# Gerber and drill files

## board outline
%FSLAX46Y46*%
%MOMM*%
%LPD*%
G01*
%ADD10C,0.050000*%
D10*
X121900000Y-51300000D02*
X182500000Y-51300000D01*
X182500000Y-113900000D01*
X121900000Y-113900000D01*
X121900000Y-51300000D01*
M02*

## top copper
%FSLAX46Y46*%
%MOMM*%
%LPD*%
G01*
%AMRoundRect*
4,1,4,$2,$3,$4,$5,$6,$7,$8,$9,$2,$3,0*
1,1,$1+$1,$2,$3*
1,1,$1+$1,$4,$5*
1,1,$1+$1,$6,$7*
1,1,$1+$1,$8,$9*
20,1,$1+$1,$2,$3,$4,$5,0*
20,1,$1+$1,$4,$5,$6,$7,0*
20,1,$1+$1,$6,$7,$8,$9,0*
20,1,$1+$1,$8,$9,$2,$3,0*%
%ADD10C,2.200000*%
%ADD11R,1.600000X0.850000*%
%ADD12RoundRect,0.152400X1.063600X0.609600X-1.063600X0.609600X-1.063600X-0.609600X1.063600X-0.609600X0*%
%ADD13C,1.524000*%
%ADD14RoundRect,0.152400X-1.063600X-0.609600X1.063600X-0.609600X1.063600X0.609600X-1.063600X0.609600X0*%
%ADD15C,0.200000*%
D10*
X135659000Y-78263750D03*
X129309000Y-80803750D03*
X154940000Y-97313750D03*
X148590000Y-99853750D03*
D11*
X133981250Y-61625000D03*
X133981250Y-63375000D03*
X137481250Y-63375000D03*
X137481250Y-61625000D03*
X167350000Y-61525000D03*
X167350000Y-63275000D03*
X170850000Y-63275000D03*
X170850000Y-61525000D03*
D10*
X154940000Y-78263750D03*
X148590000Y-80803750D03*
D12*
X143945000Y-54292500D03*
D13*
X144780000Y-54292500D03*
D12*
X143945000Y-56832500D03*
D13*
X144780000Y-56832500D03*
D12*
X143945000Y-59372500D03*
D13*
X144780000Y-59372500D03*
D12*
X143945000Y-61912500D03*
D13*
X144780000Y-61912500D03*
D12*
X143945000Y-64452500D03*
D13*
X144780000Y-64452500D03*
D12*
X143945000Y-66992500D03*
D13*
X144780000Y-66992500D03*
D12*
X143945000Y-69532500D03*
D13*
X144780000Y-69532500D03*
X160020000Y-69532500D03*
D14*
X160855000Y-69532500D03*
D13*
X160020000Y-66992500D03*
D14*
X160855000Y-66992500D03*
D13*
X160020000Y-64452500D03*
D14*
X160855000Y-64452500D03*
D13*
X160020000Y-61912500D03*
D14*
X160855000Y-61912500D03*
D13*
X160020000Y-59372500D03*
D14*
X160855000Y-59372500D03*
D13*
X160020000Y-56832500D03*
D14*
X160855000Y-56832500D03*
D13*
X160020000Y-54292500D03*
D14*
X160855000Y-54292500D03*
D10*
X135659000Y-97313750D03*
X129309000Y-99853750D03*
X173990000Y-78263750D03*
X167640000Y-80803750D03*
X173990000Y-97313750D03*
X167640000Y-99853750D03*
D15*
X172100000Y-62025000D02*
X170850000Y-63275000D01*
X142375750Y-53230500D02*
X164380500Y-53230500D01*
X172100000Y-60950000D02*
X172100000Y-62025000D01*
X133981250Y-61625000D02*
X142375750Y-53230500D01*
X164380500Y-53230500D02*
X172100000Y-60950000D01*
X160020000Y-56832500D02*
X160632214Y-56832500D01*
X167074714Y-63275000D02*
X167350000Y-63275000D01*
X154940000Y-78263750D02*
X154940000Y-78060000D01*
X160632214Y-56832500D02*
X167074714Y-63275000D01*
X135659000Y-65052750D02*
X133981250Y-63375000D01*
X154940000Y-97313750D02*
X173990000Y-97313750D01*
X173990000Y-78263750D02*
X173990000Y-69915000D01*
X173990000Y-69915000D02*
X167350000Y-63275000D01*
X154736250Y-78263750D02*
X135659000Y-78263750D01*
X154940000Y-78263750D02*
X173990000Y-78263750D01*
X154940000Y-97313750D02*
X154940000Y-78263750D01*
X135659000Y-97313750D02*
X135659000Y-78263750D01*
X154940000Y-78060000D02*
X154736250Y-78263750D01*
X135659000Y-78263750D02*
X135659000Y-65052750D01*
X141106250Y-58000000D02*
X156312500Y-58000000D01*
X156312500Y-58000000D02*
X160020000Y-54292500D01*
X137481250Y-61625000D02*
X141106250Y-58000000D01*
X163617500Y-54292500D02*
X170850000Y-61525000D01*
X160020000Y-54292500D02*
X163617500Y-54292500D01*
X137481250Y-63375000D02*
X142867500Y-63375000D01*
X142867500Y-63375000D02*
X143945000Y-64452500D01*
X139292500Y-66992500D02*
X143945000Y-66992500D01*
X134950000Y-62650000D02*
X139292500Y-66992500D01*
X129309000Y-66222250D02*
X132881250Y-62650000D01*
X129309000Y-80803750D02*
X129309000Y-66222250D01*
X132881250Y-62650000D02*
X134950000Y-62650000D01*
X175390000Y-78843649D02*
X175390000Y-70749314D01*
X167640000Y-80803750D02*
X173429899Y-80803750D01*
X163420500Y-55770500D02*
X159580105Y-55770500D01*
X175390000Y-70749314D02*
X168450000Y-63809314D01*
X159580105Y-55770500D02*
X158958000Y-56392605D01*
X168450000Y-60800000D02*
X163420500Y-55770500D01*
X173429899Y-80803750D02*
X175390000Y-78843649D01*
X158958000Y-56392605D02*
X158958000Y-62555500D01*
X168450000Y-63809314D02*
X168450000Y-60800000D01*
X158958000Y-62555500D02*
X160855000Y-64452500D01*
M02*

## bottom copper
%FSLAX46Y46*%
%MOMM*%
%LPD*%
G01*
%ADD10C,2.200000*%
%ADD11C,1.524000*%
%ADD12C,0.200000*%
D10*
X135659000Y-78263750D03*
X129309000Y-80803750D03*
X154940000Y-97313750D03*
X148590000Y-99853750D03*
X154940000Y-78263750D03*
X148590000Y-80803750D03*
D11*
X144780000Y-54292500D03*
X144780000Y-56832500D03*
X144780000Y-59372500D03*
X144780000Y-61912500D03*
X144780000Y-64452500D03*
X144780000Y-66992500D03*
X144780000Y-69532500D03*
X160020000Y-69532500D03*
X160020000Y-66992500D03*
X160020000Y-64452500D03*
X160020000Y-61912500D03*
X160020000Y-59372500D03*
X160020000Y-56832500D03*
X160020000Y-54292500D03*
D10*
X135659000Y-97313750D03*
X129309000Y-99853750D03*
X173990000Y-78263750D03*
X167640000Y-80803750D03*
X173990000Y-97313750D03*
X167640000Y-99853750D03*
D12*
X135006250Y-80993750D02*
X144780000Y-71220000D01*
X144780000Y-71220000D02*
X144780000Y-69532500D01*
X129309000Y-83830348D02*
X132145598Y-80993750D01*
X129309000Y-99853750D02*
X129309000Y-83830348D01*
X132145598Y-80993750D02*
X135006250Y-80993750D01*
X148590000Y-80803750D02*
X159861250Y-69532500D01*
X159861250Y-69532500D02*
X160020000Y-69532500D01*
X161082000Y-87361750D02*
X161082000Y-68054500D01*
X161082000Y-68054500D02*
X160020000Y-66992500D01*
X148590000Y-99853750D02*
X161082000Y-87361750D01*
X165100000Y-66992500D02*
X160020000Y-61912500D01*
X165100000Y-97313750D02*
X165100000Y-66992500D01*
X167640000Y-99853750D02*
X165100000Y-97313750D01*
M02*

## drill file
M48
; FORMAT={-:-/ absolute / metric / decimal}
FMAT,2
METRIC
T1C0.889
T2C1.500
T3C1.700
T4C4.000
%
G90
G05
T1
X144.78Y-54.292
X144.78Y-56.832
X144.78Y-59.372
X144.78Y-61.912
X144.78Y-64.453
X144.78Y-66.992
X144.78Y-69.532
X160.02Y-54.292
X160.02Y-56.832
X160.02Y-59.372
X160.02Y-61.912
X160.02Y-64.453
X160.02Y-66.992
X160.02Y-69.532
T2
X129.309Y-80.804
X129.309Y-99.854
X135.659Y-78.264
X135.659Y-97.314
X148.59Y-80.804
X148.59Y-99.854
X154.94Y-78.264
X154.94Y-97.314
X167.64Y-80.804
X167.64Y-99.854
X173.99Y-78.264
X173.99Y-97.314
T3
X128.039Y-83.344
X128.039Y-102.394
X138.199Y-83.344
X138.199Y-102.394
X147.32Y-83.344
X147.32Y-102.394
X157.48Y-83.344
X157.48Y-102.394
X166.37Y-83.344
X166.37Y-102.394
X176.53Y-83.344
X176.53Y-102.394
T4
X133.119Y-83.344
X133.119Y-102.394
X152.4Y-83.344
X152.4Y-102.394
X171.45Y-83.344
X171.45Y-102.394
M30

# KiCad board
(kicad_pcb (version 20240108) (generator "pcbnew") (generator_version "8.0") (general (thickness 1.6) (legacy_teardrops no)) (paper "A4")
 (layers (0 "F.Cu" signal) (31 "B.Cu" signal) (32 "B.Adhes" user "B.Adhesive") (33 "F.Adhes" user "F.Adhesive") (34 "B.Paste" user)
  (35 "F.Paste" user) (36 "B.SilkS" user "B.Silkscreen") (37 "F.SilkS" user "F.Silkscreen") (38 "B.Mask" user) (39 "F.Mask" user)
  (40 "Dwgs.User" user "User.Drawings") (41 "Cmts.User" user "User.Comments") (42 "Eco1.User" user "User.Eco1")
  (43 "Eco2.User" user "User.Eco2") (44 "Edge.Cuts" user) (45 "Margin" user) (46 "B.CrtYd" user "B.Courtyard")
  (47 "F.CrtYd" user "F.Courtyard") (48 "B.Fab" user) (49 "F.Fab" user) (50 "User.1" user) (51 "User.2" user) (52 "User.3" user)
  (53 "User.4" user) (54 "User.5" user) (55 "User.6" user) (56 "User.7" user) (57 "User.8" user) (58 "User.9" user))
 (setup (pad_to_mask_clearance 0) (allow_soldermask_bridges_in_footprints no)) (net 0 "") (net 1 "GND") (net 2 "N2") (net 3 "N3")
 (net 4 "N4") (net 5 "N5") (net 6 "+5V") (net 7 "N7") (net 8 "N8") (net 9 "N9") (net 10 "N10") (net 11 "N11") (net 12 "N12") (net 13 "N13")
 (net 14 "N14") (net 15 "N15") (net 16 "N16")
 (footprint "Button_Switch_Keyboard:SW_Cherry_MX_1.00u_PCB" (layer "F.Cu") (at 135.659 78.26375)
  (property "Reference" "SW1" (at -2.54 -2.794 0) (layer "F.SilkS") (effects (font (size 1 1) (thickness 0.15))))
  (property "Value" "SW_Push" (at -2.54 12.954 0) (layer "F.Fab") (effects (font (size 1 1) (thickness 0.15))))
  (pad "" np_thru_hole circle (at -7.62 5.08) (size 1.7 1.7) (drill 1.7) (layers "*.Cu" "*.Mask"))
  (pad "" np_thru_hole circle (at -2.54 5.08) (size 4 4) (drill 4) (layers "*.Cu" "*.Mask"))
  (pad "" np_thru_hole circle (at 2.54 5.08) (size 1.7 1.7) (drill 1.7) (layers "*.Cu" "*.Mask"))
  (pad "1" thru_hole circle (at 0 0) (size 2.2 2.2) (drill 1.5) (layers "*.Cu" "*.Mask") (remove_unused_layers no) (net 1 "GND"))
  (pad "2" thru_hole circle (at -6.35 2.54) (size 2.2 2.2) (drill 1.5) (layers "*.Cu" "*.Mask") (remove_unused_layers no) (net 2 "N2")))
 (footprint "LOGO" (layer "F.Cu") (at 153.1 80.9)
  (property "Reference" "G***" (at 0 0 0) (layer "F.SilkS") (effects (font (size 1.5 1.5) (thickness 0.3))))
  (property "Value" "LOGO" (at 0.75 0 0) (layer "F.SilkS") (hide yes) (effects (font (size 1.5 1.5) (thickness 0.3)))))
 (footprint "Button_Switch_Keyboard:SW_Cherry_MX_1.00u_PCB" (layer "F.Cu") (at 154.94 97.31375)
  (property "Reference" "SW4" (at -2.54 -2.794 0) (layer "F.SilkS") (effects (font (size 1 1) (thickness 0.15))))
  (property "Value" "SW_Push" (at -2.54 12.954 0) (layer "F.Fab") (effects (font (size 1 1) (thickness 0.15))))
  (pad "" np_thru_hole circle (at -7.62 5.08) (size 1.7 1.7) (drill 1.7) (layers "*.Cu" "*.Mask"))
  (pad "" np_thru_hole circle (at -2.54 5.08) (size 4 4) (drill 4) (layers "*.Cu" "*.Mask"))
  (pad "" np_thru_hole circle (at 2.54 5.08) (size 1.7 1.7) (drill 1.7) (layers "*.Cu" "*.Mask"))
  (pad "1" thru_hole circle (at 0 0) (size 2.2 2.2) (drill 1.5) (layers "*.Cu" "*.Mask") (remove_unused_layers no) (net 1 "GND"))
  (pad "2" thru_hole circle (at -6.35 2.54) (size 2.2 2.2) (drill 1.5) (layers "*.Cu" "*.Mask") (remove_unused_layers no) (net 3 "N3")))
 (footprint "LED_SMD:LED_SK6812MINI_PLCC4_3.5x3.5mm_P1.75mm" (layer "F.Cu") (at 135.73125 62.5)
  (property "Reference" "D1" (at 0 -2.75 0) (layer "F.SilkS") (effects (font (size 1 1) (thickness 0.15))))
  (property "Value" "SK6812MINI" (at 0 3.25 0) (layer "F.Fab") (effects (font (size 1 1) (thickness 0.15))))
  (pad "1" smd rect (at -1.75 -0.875) (size 1.6 0.85) (layers "F.Cu" "F.Paste" "F.Mask") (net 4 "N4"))
  (pad "2" smd rect (at -1.75 0.875) (size 1.6 0.85) (layers "F.Cu" "F.Paste" "F.Mask") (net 1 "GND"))
  (pad "3" smd rect (at 1.75 0.875) (size 1.6 0.85) (layers "F.Cu" "F.Paste" "F.Mask") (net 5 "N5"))
  (pad "4" smd rect (at 1.75 -0.875) (size 1.6 0.85) (layers "F.Cu" "F.Paste" "F.Mask") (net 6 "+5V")))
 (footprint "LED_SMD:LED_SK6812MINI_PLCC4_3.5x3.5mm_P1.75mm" (layer "F.Cu") (at 169.1 62.4)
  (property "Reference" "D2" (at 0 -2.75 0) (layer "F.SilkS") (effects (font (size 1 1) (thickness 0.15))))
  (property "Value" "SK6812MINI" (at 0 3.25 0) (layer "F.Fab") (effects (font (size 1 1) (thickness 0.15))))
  (pad "1" smd rect (at -1.75 -0.875) (size 1.6 0.85) (layers "F.Cu" "F.Paste" "F.Mask") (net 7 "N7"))
  (pad "2" smd rect (at -1.75 0.875) (size 1.6 0.85) (layers "F.Cu" "F.Paste" "F.Mask") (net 1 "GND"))
  (pad "3" smd rect (at 1.75 0.875) (size 1.6 0.85) (layers "F.Cu" "F.Paste" "F.Mask") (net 4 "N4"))
  (pad "4" smd rect (at 1.75 -0.875) (size 1.6 0.85) (layers "F.Cu" "F.Paste" "F.Mask") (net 6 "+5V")))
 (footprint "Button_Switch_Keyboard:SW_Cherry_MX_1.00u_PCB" (layer "F.Cu") (at 154.94 78.26375)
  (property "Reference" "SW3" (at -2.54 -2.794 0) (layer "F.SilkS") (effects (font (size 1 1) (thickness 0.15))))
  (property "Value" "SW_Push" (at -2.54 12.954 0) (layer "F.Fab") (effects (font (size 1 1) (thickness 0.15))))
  (pad "" np_thru_hole circle (at -7.62 5.08) (size 1.7 1.7) (drill 1.7) (layers "*.Cu" "*.Mask"))
  (pad "" np_thru_hole circle (at -2.54 5.08) (size 4 4) (drill 4) (layers "*.Cu" "*.Mask"))
  (pad "" np_thru_hole circle (at 2.54 5.08) (size 1.7 1.7) (drill 1.7) (layers "*.Cu" "*.Mask"))
  (pad "1" thru_hole circle (at 0 0) (size 2.2 2.2) (drill 1.5) (layers "*.Cu" "*.Mask") (remove_unused_layers no) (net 1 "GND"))
  (pad "2" thru_hole circle (at -6.35 2.54) (size 2.2 2.2) (drill 1.5) (layers "*.Cu" "*.Mask") (remove_unused_layers no) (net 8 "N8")))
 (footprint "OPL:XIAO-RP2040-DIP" (layer "F.Cu") (at 152.4 61.9125)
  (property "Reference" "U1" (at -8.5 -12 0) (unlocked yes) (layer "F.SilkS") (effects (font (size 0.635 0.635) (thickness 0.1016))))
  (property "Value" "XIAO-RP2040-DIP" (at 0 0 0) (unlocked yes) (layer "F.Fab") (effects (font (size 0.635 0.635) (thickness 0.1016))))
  (pad "1" smd roundrect (at -8.455 -7.62 180) (size 2.432 1.524) (layers "F.Cu" "F.Mask") (roundrect_rratio 0.1) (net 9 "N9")
   (thermal_bridge_angle 45))
  (pad "1" thru_hole circle (at -7.62 -7.62 180) (size 1.524 1.524) (drill 0.889) (layers "*.Cu" "*.Mask") (remove_unused_layers no)
   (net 9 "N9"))
  (pad "2" smd roundrect (at -8.455 -5.08 180) (size 2.432 1.524) (layers "F.Cu" "F.Mask") (roundrect_rratio 0.1) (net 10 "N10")
   (thermal_bridge_angle 45))
  (pad "2" thru_hole circle (at -7.62 -5.08 180) (size 1.524 1.524) (drill 0.889) (layers "*.Cu" "*.Mask") (remove_unused_layers no)
   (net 10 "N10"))
  (pad "3" smd roundrect (at -8.455 -2.54 180) (size 2.432 1.524) (layers "F.Cu" "F.Mask") (roundrect_rratio 0.1) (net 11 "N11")
   (thermal_bridge_angle 45))
  (pad "3" thru_hole circle (at -7.62 -2.54 180) (size 1.524 1.524) (drill 0.889) (layers "*.Cu" "*.Mask") (remove_unused_layers no)
   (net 11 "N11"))
  (pad "4" smd roundrect (at -8.455 0 180) (size 2.432 1.524) (layers "F.Cu" "F.Mask") (roundrect_rratio 0.1) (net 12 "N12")
   (thermal_bridge_angle 45))
  (pad "4" thru_hole circle (at -7.62 0 180) (size 1.524 1.524) (drill 0.889) (layers "*.Cu" "*.Mask") (remove_unused_layers no)
   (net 12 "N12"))
  (pad "5" smd roundrect (at -8.455 2.54 180) (size 2.432 1.524) (layers "F.Cu" "F.Mask") (roundrect_rratio 0.1) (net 5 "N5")
   (thermal_bridge_angle 45))
  (pad "5" thru_hole circle (at -7.62 2.54 180) (size 1.524 1.524) (drill 0.889) (layers "*.Cu" "*.Mask") (remove_unused_layers no)
   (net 5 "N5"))
  (pad "6" smd roundrect (at -8.455 5.08 180) (size 2.432 1.524) (layers "F.Cu" "F.Mask") (roundrect_rratio 0.1) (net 2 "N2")
   (thermal_bridge_angle 45))
  (pad "6" thru_hole circle (at -7.62 5.08 180) (size 1.524 1.524) (drill 0.889) (layers "*.Cu" "*.Mask") (remove_unused_layers no)
   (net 2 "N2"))
  (pad "7" smd roundrect (at -8.455 7.62 180) (size 2.432 1.524) (layers "F.Cu" "F.Mask") (roundrect_rratio 0.1) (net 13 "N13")
   (thermal_bridge_angle 45))
  (pad "7" thru_hole circle (at -7.62 7.62 180) (size 1.524 1.524) (drill 0.889) (layers "*.Cu" "*.Mask") (remove_unused_layers no)
   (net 13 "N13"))
  (pad "8" thru_hole circle (at 7.62 7.62) (size 1.524 1.524) (drill 0.889) (layers "*.Cu" "*.Mask") (remove_unused_layers no) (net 8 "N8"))
  (pad "8" smd roundrect (at 8.455 7.62) (size 2.432 1.524) (layers "F.Cu" "F.Mask") (roundrect_rratio 0.1) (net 8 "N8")
   (thermal_bridge_angle 45))
  (pad "9" thru_hole circle (at 7.62 5.08) (size 1.524 1.524) (drill 0.889) (layers "*.Cu" "*.Mask") (remove_unused_layers no) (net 3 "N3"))
  (pad "9" smd roundrect (at 8.455 5.08) (size 2.432 1.524) (layers "F.Cu" "F.Mask") (roundrect_rratio 0.1) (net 3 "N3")
   (thermal_bridge_angle 45))
  (pad "10" thru_hole circle (at 7.62 2.54) (size 1.524 1.524) (drill 0.889) (layers "*.Cu" "*.Mask") (remove_unused_layers no)
   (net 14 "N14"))
  (pad "10" smd roundrect (at 8.455 2.54) (size 2.432 1.524) (layers "F.Cu" "F.Mask") (roundrect_rratio 0.1) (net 14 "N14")
   (thermal_bridge_angle 45))
  (pad "11" thru_hole circle (at 7.62 0) (size 1.524 1.524) (drill 0.889) (layers "*.Cu" "*.Mask") (remove_unused_layers no) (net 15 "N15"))
  (pad "11" smd roundrect (at 8.455 0) (size 2.432 1.524) (layers "F.Cu" "F.Mask") (roundrect_rratio 0.1) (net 15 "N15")
   (thermal_bridge_angle 45))
  (pad "12" thru_hole circle (at 7.62 -2.54) (size 1.524 1.524) (drill 0.889) (layers "*.Cu" "*.Mask") (remove_unused_layers no)
   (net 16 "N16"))
  (pad "12" smd roundrect (at 8.455 -2.54) (size 2.432 1.524) (layers "F.Cu" "F.Mask") (roundrect_rratio 0.1) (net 16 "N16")
   (thermal_bridge_angle 45))
  (pad "13" thru_hole circle (at 7.62 -5.08) (size 1.524 1.524) (drill 0.889) (layers "*.Cu" "*.Mask") (remove_unused_layers no)
   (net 1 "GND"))
  (pad "13" smd roundrect (at 8.455 -5.08) (size 2.432 1.524) (layers "F.Cu" "F.Mask") (roundrect_rratio 0.1) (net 1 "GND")
   (thermal_bridge_angle 45))
  (pad "14" thru_hole circle (at 7.62 -7.62) (size 1.524 1.524) (drill 0.889) (layers "*.Cu" "*.Mask") (remove_unused_layers no)
   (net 6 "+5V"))
  (pad "14" smd roundrect (at 8.455 -7.62) (size 2.432 1.524) (layers "F.Cu" "F.Mask") (roundrect_rratio 0.1) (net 6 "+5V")
   (thermal_bridge_angle 45)))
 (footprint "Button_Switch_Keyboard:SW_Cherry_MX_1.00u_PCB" (layer "F.Cu") (at 135.659 97.31375)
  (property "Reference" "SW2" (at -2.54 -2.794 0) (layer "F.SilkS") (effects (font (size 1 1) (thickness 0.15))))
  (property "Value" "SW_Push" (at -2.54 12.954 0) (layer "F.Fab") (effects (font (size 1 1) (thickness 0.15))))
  (pad "" np_thru_hole circle (at -7.62 5.08) (size 1.7 1.7) (drill 1.7) (layers "*.Cu" "*.Mask"))
  (pad "" np_thru_hole circle (at -2.54 5.08) (size 4 4) (drill 4) (layers "*.Cu" "*.Mask"))
  (pad "" np_thru_hole circle (at 2.54 5.08) (size 1.7 1.7) (drill 1.7) (layers "*.Cu" "*.Mask"))
  (pad "1" thru_hole circle (at 0 0) (size 2.2 2.2) (drill 1.5) (layers "*.Cu" "*.Mask") (remove_unused_layers no) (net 1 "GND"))
  (pad "2" thru_hole circle (at -6.35 2.54) (size 2.2 2.2) (drill 1.5) (layers "*.Cu" "*.Mask") (remove_unused_layers no) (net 13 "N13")))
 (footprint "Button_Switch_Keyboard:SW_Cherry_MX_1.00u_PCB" (layer "F.Cu") (at 173.99 78.26375)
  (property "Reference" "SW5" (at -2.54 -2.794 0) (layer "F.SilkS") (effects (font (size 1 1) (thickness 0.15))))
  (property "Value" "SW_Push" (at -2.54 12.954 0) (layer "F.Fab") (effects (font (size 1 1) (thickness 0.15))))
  (pad "" np_thru_hole circle (at -7.62 5.08) (size 1.7 1.7) (drill 1.7) (layers "*.Cu" "*.Mask"))
  (pad "" np_thru_hole circle (at -2.54 5.08) (size 4 4) (drill 4) (layers "*.Cu" "*.Mask"))
  (pad "" np_thru_hole circle (at 2.54 5.08) (size 1.7 1.7) (drill 1.7) (layers "*.Cu" "*.Mask"))
  (pad "1" thru_hole circle (at 0 0) (size 2.2 2.2) (drill 1.5) (layers "*.Cu" "*.Mask") (remove_unused_layers no) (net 1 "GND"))
  (pad "2" thru_hole circle (at -6.35 2.54) (size 2.2 2.2) (drill 1.5) (layers "*.Cu" "*.Mask") (remove_unused_layers no) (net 14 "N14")))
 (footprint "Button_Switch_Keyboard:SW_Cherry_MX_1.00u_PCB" (layer "F.Cu") (at 173.99 97.31375)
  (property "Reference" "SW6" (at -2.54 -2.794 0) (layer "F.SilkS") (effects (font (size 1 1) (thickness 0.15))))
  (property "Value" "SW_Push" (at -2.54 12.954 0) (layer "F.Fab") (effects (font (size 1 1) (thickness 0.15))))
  (pad "" np_thru_hole circle (at -7.62 5.08) (size 1.7 1.7) (drill 1.7) (layers "*.Cu" "*.Mask"))
  (pad "" np_thru_hole circle (at -2.54 5.08) (size 4 4) (drill 4) (layers "*.Cu" "*.Mask"))
  (pad "" np_thru_hole circle (at 2.54 5.08) (size 1.7 1.7) (drill 1.7) (layers "*.Cu" "*.Mask"))
  (pad "1" thru_hole circle (at 0 0) (size 2.2 2.2) (drill 1.5) (layers "*.Cu" "*.Mask") (remove_unused_layers no) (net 1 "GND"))
  (pad "2" thru_hole circle (at -6.35 2.54) (size 2.2 2.2) (drill 1.5) (layers "*.Cu" "*.Mask") (remove_unused_layers no) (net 15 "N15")))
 (gr_rect (start 121.9 51.3) (end 182.5 113.9) (stroke (width 0.05) (type default)) (fill none) (layer "Edge.Cuts"))
 (segment (start 172.1 62.025) (end 170.85 63.275) (width 0.2) (layer "F.Cu") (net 4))
 (segment (start 142.37575 53.2305) (end 164.3805 53.2305) (width 0.2) (layer "F.Cu") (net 4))
 (segment (start 172.1 60.95) (end 172.1 62.025) (width 0.2) (layer "F.Cu") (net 4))
 (segment (start 133.98125 61.625) (end 142.37575 53.2305) (width 0.2) (layer "F.Cu") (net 4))
 (segment (start 164.3805 53.2305) (end 172.1 60.95) (width 0.2) (layer "F.Cu") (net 4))
 (segment (start 160.02 56.8325) (end 160.632214 56.8325) (width 0.2) (layer "F.Cu") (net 1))
 (segment (start 167.074714 63.275) (end 167.35 63.275) (width 0.2) (layer "F.Cu") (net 1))
 (segment (start 154.94 78.26375) (end 154.94 78.06) (width 0.2) (layer "F.Cu") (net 1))
 (segment (start 160.632214 56.8325) (end 167.074714 63.275) (width 0.2) (layer "F.Cu") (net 1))
 (segment (start 135.659 65.05275) (end 133.98125 63.375) (width 0.2) (layer "F.Cu") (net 1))
 (segment (start 154.94 97.31375) (end 173.99 97.31375) (width 0.2) (layer "F.Cu") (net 1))
 (segment (start 173.99 78.26375) (end 173.99 69.915) (width 0.2) (layer "F.Cu") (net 1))
 (segment (start 173.99 69.915) (end 167.35 63.275) (width 0.2) (layer "F.Cu") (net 1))
 (segment (start 154.73625 78.26375) (end 135.659 78.26375) (width 0.2) (layer "F.Cu") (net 1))
 (segment (start 154.94 78.26375) (end 173.99 78.26375) (width 0.2) (layer "F.Cu") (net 1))
 (segment (start 154.94 97.31375) (end 154.94 78.26375) (width 0.2) (layer "F.Cu") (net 1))
 (segment (start 135.659 97.31375) (end 135.659 78.26375) (width 0.2) (layer "F.Cu") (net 1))
 (segment (start 154.94 78.06) (end 154.73625 78.26375) (width 0.2) (layer "F.Cu") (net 1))
 (segment (start 135.659 78.26375) (end 135.659 65.05275) (width 0.2) (layer "F.Cu") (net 1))
 (segment (start 141.10625 58) (end 156.3125 58) (width 0.2) (layer "F.Cu") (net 6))
 (segment (start 156.3125 58) (end 160.02 54.2925) (width 0.2) (layer "F.Cu") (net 6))
 (segment (start 137.48125 61.625) (end 141.10625 58) (width 0.2) (layer "F.Cu") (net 6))
 (segment (start 163.6175 54.2925) (end 170.85 61.525) (width 0.2) (layer "F.Cu") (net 6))
 (segment (start 160.02 54.2925) (end 163.6175 54.2925) (width 0.2) (layer "F.Cu") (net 6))
 (segment (start 137.48125 63.375) (end 142.8675 63.375) (width 0.2) (layer "F.Cu") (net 5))
 (segment (start 142.8675 63.375) (end 143.945 64.4525) (width 0.2) (layer "F.Cu") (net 5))
 (segment (start 139.2925 66.9925) (end 143.945 66.9925) (width 0.2) (layer "F.Cu") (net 2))
 (segment (start 134.95 62.65) (end 139.2925 66.9925) (width 0.2) (layer "F.Cu") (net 2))
 (segment (start 129.309 66.22225) (end 132.88125 62.65) (width 0.2) (layer "F.Cu") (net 2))
 (segment (start 129.309 80.80375) (end 129.309 66.22225) (width 0.2) (layer "F.Cu") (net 2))
 (segment (start 132.88125 62.65) (end 134.95 62.65) (width 0.2) (layer "F.Cu") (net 2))
 (segment (start 135.00625 80.99375) (end 144.78 71.22) (width 0.2) (layer "B.Cu") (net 13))
 (segment (start 144.78 71.22) (end 144.78 69.5325) (width 0.2) (layer "B.Cu") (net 13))
 (segment (start 129.309 83.830348) (end 132.145598 80.99375) (width 0.2) (layer "B.Cu") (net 13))
 (segment (start 129.309 99.85375) (end 129.309 83.830348) (width 0.2) (layer "B.Cu") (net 13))
 (segment (start 132.145598 80.99375) (end 135.00625 80.99375) (width 0.2) (layer "B.Cu") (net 13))
 (segment (start 148.59 80.80375) (end 159.86125 69.5325) (width 0.2) (layer "B.Cu") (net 8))
 (segment (start 159.86125 69.5325) (end 160.02 69.5325) (width 0.2) (layer "B.Cu") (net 8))
 (segment (start 161.082 87.36175) (end 161.082 68.0545) (width 0.2) (layer "B.Cu") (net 3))
 (segment (start 161.082 68.0545) (end 160.02 66.9925) (width 0.2) (layer "B.Cu") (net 3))
 (segment (start 148.59 99.85375) (end 161.082 87.36175) (width 0.2) (layer "B.Cu") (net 3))
 (segment (start 175.39 78.843649) (end 175.39 70.749314) (width 0.2) (layer "F.Cu") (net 14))
 (segment (start 167.64 80.80375) (end 173.429899 80.80375) (width 0.2) (layer "F.Cu") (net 14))
 (segment (start 163.4205 55.7705) (end 159.580105 55.7705) (width 0.2) (layer "F.Cu") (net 14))
 (segment (start 175.39 70.749314) (end 168.45 63.809314) (width 0.2) (layer "F.Cu") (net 14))
 (segment (start 159.580105 55.7705) (end 158.958 56.392605) (width 0.2) (layer "F.Cu") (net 14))
 (segment (start 168.45 60.8) (end 163.4205 55.7705) (width 0.2) (layer "F.Cu") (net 14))
 (segment (start 173.429899 80.80375) (end 175.39 78.843649) (width 0.2) (layer "F.Cu") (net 14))
 (segment (start 158.958 56.392605) (end 158.958 62.5555) (width 0.2) (layer "F.Cu") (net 14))
 (segment (start 168.45 63.809314) (end 168.45 60.8) (width 0.2) (layer "F.Cu") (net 14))
 (segment (start 158.958 62.5555) (end 160.855 64.4525) (width 0.2) (layer "F.Cu") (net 14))
 (segment (start 165.1 66.9925) (end 160.02 61.9125) (width 0.2) (layer "B.Cu") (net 15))
 (segment (start 165.1 97.31375) (end 165.1 66.9925) (width 0.2) (layer "B.Cu") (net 15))
 (segment (start 167.64 99.85375) (end 165.1 97.31375) (width 0.2) (layer "B.Cu") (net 15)))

